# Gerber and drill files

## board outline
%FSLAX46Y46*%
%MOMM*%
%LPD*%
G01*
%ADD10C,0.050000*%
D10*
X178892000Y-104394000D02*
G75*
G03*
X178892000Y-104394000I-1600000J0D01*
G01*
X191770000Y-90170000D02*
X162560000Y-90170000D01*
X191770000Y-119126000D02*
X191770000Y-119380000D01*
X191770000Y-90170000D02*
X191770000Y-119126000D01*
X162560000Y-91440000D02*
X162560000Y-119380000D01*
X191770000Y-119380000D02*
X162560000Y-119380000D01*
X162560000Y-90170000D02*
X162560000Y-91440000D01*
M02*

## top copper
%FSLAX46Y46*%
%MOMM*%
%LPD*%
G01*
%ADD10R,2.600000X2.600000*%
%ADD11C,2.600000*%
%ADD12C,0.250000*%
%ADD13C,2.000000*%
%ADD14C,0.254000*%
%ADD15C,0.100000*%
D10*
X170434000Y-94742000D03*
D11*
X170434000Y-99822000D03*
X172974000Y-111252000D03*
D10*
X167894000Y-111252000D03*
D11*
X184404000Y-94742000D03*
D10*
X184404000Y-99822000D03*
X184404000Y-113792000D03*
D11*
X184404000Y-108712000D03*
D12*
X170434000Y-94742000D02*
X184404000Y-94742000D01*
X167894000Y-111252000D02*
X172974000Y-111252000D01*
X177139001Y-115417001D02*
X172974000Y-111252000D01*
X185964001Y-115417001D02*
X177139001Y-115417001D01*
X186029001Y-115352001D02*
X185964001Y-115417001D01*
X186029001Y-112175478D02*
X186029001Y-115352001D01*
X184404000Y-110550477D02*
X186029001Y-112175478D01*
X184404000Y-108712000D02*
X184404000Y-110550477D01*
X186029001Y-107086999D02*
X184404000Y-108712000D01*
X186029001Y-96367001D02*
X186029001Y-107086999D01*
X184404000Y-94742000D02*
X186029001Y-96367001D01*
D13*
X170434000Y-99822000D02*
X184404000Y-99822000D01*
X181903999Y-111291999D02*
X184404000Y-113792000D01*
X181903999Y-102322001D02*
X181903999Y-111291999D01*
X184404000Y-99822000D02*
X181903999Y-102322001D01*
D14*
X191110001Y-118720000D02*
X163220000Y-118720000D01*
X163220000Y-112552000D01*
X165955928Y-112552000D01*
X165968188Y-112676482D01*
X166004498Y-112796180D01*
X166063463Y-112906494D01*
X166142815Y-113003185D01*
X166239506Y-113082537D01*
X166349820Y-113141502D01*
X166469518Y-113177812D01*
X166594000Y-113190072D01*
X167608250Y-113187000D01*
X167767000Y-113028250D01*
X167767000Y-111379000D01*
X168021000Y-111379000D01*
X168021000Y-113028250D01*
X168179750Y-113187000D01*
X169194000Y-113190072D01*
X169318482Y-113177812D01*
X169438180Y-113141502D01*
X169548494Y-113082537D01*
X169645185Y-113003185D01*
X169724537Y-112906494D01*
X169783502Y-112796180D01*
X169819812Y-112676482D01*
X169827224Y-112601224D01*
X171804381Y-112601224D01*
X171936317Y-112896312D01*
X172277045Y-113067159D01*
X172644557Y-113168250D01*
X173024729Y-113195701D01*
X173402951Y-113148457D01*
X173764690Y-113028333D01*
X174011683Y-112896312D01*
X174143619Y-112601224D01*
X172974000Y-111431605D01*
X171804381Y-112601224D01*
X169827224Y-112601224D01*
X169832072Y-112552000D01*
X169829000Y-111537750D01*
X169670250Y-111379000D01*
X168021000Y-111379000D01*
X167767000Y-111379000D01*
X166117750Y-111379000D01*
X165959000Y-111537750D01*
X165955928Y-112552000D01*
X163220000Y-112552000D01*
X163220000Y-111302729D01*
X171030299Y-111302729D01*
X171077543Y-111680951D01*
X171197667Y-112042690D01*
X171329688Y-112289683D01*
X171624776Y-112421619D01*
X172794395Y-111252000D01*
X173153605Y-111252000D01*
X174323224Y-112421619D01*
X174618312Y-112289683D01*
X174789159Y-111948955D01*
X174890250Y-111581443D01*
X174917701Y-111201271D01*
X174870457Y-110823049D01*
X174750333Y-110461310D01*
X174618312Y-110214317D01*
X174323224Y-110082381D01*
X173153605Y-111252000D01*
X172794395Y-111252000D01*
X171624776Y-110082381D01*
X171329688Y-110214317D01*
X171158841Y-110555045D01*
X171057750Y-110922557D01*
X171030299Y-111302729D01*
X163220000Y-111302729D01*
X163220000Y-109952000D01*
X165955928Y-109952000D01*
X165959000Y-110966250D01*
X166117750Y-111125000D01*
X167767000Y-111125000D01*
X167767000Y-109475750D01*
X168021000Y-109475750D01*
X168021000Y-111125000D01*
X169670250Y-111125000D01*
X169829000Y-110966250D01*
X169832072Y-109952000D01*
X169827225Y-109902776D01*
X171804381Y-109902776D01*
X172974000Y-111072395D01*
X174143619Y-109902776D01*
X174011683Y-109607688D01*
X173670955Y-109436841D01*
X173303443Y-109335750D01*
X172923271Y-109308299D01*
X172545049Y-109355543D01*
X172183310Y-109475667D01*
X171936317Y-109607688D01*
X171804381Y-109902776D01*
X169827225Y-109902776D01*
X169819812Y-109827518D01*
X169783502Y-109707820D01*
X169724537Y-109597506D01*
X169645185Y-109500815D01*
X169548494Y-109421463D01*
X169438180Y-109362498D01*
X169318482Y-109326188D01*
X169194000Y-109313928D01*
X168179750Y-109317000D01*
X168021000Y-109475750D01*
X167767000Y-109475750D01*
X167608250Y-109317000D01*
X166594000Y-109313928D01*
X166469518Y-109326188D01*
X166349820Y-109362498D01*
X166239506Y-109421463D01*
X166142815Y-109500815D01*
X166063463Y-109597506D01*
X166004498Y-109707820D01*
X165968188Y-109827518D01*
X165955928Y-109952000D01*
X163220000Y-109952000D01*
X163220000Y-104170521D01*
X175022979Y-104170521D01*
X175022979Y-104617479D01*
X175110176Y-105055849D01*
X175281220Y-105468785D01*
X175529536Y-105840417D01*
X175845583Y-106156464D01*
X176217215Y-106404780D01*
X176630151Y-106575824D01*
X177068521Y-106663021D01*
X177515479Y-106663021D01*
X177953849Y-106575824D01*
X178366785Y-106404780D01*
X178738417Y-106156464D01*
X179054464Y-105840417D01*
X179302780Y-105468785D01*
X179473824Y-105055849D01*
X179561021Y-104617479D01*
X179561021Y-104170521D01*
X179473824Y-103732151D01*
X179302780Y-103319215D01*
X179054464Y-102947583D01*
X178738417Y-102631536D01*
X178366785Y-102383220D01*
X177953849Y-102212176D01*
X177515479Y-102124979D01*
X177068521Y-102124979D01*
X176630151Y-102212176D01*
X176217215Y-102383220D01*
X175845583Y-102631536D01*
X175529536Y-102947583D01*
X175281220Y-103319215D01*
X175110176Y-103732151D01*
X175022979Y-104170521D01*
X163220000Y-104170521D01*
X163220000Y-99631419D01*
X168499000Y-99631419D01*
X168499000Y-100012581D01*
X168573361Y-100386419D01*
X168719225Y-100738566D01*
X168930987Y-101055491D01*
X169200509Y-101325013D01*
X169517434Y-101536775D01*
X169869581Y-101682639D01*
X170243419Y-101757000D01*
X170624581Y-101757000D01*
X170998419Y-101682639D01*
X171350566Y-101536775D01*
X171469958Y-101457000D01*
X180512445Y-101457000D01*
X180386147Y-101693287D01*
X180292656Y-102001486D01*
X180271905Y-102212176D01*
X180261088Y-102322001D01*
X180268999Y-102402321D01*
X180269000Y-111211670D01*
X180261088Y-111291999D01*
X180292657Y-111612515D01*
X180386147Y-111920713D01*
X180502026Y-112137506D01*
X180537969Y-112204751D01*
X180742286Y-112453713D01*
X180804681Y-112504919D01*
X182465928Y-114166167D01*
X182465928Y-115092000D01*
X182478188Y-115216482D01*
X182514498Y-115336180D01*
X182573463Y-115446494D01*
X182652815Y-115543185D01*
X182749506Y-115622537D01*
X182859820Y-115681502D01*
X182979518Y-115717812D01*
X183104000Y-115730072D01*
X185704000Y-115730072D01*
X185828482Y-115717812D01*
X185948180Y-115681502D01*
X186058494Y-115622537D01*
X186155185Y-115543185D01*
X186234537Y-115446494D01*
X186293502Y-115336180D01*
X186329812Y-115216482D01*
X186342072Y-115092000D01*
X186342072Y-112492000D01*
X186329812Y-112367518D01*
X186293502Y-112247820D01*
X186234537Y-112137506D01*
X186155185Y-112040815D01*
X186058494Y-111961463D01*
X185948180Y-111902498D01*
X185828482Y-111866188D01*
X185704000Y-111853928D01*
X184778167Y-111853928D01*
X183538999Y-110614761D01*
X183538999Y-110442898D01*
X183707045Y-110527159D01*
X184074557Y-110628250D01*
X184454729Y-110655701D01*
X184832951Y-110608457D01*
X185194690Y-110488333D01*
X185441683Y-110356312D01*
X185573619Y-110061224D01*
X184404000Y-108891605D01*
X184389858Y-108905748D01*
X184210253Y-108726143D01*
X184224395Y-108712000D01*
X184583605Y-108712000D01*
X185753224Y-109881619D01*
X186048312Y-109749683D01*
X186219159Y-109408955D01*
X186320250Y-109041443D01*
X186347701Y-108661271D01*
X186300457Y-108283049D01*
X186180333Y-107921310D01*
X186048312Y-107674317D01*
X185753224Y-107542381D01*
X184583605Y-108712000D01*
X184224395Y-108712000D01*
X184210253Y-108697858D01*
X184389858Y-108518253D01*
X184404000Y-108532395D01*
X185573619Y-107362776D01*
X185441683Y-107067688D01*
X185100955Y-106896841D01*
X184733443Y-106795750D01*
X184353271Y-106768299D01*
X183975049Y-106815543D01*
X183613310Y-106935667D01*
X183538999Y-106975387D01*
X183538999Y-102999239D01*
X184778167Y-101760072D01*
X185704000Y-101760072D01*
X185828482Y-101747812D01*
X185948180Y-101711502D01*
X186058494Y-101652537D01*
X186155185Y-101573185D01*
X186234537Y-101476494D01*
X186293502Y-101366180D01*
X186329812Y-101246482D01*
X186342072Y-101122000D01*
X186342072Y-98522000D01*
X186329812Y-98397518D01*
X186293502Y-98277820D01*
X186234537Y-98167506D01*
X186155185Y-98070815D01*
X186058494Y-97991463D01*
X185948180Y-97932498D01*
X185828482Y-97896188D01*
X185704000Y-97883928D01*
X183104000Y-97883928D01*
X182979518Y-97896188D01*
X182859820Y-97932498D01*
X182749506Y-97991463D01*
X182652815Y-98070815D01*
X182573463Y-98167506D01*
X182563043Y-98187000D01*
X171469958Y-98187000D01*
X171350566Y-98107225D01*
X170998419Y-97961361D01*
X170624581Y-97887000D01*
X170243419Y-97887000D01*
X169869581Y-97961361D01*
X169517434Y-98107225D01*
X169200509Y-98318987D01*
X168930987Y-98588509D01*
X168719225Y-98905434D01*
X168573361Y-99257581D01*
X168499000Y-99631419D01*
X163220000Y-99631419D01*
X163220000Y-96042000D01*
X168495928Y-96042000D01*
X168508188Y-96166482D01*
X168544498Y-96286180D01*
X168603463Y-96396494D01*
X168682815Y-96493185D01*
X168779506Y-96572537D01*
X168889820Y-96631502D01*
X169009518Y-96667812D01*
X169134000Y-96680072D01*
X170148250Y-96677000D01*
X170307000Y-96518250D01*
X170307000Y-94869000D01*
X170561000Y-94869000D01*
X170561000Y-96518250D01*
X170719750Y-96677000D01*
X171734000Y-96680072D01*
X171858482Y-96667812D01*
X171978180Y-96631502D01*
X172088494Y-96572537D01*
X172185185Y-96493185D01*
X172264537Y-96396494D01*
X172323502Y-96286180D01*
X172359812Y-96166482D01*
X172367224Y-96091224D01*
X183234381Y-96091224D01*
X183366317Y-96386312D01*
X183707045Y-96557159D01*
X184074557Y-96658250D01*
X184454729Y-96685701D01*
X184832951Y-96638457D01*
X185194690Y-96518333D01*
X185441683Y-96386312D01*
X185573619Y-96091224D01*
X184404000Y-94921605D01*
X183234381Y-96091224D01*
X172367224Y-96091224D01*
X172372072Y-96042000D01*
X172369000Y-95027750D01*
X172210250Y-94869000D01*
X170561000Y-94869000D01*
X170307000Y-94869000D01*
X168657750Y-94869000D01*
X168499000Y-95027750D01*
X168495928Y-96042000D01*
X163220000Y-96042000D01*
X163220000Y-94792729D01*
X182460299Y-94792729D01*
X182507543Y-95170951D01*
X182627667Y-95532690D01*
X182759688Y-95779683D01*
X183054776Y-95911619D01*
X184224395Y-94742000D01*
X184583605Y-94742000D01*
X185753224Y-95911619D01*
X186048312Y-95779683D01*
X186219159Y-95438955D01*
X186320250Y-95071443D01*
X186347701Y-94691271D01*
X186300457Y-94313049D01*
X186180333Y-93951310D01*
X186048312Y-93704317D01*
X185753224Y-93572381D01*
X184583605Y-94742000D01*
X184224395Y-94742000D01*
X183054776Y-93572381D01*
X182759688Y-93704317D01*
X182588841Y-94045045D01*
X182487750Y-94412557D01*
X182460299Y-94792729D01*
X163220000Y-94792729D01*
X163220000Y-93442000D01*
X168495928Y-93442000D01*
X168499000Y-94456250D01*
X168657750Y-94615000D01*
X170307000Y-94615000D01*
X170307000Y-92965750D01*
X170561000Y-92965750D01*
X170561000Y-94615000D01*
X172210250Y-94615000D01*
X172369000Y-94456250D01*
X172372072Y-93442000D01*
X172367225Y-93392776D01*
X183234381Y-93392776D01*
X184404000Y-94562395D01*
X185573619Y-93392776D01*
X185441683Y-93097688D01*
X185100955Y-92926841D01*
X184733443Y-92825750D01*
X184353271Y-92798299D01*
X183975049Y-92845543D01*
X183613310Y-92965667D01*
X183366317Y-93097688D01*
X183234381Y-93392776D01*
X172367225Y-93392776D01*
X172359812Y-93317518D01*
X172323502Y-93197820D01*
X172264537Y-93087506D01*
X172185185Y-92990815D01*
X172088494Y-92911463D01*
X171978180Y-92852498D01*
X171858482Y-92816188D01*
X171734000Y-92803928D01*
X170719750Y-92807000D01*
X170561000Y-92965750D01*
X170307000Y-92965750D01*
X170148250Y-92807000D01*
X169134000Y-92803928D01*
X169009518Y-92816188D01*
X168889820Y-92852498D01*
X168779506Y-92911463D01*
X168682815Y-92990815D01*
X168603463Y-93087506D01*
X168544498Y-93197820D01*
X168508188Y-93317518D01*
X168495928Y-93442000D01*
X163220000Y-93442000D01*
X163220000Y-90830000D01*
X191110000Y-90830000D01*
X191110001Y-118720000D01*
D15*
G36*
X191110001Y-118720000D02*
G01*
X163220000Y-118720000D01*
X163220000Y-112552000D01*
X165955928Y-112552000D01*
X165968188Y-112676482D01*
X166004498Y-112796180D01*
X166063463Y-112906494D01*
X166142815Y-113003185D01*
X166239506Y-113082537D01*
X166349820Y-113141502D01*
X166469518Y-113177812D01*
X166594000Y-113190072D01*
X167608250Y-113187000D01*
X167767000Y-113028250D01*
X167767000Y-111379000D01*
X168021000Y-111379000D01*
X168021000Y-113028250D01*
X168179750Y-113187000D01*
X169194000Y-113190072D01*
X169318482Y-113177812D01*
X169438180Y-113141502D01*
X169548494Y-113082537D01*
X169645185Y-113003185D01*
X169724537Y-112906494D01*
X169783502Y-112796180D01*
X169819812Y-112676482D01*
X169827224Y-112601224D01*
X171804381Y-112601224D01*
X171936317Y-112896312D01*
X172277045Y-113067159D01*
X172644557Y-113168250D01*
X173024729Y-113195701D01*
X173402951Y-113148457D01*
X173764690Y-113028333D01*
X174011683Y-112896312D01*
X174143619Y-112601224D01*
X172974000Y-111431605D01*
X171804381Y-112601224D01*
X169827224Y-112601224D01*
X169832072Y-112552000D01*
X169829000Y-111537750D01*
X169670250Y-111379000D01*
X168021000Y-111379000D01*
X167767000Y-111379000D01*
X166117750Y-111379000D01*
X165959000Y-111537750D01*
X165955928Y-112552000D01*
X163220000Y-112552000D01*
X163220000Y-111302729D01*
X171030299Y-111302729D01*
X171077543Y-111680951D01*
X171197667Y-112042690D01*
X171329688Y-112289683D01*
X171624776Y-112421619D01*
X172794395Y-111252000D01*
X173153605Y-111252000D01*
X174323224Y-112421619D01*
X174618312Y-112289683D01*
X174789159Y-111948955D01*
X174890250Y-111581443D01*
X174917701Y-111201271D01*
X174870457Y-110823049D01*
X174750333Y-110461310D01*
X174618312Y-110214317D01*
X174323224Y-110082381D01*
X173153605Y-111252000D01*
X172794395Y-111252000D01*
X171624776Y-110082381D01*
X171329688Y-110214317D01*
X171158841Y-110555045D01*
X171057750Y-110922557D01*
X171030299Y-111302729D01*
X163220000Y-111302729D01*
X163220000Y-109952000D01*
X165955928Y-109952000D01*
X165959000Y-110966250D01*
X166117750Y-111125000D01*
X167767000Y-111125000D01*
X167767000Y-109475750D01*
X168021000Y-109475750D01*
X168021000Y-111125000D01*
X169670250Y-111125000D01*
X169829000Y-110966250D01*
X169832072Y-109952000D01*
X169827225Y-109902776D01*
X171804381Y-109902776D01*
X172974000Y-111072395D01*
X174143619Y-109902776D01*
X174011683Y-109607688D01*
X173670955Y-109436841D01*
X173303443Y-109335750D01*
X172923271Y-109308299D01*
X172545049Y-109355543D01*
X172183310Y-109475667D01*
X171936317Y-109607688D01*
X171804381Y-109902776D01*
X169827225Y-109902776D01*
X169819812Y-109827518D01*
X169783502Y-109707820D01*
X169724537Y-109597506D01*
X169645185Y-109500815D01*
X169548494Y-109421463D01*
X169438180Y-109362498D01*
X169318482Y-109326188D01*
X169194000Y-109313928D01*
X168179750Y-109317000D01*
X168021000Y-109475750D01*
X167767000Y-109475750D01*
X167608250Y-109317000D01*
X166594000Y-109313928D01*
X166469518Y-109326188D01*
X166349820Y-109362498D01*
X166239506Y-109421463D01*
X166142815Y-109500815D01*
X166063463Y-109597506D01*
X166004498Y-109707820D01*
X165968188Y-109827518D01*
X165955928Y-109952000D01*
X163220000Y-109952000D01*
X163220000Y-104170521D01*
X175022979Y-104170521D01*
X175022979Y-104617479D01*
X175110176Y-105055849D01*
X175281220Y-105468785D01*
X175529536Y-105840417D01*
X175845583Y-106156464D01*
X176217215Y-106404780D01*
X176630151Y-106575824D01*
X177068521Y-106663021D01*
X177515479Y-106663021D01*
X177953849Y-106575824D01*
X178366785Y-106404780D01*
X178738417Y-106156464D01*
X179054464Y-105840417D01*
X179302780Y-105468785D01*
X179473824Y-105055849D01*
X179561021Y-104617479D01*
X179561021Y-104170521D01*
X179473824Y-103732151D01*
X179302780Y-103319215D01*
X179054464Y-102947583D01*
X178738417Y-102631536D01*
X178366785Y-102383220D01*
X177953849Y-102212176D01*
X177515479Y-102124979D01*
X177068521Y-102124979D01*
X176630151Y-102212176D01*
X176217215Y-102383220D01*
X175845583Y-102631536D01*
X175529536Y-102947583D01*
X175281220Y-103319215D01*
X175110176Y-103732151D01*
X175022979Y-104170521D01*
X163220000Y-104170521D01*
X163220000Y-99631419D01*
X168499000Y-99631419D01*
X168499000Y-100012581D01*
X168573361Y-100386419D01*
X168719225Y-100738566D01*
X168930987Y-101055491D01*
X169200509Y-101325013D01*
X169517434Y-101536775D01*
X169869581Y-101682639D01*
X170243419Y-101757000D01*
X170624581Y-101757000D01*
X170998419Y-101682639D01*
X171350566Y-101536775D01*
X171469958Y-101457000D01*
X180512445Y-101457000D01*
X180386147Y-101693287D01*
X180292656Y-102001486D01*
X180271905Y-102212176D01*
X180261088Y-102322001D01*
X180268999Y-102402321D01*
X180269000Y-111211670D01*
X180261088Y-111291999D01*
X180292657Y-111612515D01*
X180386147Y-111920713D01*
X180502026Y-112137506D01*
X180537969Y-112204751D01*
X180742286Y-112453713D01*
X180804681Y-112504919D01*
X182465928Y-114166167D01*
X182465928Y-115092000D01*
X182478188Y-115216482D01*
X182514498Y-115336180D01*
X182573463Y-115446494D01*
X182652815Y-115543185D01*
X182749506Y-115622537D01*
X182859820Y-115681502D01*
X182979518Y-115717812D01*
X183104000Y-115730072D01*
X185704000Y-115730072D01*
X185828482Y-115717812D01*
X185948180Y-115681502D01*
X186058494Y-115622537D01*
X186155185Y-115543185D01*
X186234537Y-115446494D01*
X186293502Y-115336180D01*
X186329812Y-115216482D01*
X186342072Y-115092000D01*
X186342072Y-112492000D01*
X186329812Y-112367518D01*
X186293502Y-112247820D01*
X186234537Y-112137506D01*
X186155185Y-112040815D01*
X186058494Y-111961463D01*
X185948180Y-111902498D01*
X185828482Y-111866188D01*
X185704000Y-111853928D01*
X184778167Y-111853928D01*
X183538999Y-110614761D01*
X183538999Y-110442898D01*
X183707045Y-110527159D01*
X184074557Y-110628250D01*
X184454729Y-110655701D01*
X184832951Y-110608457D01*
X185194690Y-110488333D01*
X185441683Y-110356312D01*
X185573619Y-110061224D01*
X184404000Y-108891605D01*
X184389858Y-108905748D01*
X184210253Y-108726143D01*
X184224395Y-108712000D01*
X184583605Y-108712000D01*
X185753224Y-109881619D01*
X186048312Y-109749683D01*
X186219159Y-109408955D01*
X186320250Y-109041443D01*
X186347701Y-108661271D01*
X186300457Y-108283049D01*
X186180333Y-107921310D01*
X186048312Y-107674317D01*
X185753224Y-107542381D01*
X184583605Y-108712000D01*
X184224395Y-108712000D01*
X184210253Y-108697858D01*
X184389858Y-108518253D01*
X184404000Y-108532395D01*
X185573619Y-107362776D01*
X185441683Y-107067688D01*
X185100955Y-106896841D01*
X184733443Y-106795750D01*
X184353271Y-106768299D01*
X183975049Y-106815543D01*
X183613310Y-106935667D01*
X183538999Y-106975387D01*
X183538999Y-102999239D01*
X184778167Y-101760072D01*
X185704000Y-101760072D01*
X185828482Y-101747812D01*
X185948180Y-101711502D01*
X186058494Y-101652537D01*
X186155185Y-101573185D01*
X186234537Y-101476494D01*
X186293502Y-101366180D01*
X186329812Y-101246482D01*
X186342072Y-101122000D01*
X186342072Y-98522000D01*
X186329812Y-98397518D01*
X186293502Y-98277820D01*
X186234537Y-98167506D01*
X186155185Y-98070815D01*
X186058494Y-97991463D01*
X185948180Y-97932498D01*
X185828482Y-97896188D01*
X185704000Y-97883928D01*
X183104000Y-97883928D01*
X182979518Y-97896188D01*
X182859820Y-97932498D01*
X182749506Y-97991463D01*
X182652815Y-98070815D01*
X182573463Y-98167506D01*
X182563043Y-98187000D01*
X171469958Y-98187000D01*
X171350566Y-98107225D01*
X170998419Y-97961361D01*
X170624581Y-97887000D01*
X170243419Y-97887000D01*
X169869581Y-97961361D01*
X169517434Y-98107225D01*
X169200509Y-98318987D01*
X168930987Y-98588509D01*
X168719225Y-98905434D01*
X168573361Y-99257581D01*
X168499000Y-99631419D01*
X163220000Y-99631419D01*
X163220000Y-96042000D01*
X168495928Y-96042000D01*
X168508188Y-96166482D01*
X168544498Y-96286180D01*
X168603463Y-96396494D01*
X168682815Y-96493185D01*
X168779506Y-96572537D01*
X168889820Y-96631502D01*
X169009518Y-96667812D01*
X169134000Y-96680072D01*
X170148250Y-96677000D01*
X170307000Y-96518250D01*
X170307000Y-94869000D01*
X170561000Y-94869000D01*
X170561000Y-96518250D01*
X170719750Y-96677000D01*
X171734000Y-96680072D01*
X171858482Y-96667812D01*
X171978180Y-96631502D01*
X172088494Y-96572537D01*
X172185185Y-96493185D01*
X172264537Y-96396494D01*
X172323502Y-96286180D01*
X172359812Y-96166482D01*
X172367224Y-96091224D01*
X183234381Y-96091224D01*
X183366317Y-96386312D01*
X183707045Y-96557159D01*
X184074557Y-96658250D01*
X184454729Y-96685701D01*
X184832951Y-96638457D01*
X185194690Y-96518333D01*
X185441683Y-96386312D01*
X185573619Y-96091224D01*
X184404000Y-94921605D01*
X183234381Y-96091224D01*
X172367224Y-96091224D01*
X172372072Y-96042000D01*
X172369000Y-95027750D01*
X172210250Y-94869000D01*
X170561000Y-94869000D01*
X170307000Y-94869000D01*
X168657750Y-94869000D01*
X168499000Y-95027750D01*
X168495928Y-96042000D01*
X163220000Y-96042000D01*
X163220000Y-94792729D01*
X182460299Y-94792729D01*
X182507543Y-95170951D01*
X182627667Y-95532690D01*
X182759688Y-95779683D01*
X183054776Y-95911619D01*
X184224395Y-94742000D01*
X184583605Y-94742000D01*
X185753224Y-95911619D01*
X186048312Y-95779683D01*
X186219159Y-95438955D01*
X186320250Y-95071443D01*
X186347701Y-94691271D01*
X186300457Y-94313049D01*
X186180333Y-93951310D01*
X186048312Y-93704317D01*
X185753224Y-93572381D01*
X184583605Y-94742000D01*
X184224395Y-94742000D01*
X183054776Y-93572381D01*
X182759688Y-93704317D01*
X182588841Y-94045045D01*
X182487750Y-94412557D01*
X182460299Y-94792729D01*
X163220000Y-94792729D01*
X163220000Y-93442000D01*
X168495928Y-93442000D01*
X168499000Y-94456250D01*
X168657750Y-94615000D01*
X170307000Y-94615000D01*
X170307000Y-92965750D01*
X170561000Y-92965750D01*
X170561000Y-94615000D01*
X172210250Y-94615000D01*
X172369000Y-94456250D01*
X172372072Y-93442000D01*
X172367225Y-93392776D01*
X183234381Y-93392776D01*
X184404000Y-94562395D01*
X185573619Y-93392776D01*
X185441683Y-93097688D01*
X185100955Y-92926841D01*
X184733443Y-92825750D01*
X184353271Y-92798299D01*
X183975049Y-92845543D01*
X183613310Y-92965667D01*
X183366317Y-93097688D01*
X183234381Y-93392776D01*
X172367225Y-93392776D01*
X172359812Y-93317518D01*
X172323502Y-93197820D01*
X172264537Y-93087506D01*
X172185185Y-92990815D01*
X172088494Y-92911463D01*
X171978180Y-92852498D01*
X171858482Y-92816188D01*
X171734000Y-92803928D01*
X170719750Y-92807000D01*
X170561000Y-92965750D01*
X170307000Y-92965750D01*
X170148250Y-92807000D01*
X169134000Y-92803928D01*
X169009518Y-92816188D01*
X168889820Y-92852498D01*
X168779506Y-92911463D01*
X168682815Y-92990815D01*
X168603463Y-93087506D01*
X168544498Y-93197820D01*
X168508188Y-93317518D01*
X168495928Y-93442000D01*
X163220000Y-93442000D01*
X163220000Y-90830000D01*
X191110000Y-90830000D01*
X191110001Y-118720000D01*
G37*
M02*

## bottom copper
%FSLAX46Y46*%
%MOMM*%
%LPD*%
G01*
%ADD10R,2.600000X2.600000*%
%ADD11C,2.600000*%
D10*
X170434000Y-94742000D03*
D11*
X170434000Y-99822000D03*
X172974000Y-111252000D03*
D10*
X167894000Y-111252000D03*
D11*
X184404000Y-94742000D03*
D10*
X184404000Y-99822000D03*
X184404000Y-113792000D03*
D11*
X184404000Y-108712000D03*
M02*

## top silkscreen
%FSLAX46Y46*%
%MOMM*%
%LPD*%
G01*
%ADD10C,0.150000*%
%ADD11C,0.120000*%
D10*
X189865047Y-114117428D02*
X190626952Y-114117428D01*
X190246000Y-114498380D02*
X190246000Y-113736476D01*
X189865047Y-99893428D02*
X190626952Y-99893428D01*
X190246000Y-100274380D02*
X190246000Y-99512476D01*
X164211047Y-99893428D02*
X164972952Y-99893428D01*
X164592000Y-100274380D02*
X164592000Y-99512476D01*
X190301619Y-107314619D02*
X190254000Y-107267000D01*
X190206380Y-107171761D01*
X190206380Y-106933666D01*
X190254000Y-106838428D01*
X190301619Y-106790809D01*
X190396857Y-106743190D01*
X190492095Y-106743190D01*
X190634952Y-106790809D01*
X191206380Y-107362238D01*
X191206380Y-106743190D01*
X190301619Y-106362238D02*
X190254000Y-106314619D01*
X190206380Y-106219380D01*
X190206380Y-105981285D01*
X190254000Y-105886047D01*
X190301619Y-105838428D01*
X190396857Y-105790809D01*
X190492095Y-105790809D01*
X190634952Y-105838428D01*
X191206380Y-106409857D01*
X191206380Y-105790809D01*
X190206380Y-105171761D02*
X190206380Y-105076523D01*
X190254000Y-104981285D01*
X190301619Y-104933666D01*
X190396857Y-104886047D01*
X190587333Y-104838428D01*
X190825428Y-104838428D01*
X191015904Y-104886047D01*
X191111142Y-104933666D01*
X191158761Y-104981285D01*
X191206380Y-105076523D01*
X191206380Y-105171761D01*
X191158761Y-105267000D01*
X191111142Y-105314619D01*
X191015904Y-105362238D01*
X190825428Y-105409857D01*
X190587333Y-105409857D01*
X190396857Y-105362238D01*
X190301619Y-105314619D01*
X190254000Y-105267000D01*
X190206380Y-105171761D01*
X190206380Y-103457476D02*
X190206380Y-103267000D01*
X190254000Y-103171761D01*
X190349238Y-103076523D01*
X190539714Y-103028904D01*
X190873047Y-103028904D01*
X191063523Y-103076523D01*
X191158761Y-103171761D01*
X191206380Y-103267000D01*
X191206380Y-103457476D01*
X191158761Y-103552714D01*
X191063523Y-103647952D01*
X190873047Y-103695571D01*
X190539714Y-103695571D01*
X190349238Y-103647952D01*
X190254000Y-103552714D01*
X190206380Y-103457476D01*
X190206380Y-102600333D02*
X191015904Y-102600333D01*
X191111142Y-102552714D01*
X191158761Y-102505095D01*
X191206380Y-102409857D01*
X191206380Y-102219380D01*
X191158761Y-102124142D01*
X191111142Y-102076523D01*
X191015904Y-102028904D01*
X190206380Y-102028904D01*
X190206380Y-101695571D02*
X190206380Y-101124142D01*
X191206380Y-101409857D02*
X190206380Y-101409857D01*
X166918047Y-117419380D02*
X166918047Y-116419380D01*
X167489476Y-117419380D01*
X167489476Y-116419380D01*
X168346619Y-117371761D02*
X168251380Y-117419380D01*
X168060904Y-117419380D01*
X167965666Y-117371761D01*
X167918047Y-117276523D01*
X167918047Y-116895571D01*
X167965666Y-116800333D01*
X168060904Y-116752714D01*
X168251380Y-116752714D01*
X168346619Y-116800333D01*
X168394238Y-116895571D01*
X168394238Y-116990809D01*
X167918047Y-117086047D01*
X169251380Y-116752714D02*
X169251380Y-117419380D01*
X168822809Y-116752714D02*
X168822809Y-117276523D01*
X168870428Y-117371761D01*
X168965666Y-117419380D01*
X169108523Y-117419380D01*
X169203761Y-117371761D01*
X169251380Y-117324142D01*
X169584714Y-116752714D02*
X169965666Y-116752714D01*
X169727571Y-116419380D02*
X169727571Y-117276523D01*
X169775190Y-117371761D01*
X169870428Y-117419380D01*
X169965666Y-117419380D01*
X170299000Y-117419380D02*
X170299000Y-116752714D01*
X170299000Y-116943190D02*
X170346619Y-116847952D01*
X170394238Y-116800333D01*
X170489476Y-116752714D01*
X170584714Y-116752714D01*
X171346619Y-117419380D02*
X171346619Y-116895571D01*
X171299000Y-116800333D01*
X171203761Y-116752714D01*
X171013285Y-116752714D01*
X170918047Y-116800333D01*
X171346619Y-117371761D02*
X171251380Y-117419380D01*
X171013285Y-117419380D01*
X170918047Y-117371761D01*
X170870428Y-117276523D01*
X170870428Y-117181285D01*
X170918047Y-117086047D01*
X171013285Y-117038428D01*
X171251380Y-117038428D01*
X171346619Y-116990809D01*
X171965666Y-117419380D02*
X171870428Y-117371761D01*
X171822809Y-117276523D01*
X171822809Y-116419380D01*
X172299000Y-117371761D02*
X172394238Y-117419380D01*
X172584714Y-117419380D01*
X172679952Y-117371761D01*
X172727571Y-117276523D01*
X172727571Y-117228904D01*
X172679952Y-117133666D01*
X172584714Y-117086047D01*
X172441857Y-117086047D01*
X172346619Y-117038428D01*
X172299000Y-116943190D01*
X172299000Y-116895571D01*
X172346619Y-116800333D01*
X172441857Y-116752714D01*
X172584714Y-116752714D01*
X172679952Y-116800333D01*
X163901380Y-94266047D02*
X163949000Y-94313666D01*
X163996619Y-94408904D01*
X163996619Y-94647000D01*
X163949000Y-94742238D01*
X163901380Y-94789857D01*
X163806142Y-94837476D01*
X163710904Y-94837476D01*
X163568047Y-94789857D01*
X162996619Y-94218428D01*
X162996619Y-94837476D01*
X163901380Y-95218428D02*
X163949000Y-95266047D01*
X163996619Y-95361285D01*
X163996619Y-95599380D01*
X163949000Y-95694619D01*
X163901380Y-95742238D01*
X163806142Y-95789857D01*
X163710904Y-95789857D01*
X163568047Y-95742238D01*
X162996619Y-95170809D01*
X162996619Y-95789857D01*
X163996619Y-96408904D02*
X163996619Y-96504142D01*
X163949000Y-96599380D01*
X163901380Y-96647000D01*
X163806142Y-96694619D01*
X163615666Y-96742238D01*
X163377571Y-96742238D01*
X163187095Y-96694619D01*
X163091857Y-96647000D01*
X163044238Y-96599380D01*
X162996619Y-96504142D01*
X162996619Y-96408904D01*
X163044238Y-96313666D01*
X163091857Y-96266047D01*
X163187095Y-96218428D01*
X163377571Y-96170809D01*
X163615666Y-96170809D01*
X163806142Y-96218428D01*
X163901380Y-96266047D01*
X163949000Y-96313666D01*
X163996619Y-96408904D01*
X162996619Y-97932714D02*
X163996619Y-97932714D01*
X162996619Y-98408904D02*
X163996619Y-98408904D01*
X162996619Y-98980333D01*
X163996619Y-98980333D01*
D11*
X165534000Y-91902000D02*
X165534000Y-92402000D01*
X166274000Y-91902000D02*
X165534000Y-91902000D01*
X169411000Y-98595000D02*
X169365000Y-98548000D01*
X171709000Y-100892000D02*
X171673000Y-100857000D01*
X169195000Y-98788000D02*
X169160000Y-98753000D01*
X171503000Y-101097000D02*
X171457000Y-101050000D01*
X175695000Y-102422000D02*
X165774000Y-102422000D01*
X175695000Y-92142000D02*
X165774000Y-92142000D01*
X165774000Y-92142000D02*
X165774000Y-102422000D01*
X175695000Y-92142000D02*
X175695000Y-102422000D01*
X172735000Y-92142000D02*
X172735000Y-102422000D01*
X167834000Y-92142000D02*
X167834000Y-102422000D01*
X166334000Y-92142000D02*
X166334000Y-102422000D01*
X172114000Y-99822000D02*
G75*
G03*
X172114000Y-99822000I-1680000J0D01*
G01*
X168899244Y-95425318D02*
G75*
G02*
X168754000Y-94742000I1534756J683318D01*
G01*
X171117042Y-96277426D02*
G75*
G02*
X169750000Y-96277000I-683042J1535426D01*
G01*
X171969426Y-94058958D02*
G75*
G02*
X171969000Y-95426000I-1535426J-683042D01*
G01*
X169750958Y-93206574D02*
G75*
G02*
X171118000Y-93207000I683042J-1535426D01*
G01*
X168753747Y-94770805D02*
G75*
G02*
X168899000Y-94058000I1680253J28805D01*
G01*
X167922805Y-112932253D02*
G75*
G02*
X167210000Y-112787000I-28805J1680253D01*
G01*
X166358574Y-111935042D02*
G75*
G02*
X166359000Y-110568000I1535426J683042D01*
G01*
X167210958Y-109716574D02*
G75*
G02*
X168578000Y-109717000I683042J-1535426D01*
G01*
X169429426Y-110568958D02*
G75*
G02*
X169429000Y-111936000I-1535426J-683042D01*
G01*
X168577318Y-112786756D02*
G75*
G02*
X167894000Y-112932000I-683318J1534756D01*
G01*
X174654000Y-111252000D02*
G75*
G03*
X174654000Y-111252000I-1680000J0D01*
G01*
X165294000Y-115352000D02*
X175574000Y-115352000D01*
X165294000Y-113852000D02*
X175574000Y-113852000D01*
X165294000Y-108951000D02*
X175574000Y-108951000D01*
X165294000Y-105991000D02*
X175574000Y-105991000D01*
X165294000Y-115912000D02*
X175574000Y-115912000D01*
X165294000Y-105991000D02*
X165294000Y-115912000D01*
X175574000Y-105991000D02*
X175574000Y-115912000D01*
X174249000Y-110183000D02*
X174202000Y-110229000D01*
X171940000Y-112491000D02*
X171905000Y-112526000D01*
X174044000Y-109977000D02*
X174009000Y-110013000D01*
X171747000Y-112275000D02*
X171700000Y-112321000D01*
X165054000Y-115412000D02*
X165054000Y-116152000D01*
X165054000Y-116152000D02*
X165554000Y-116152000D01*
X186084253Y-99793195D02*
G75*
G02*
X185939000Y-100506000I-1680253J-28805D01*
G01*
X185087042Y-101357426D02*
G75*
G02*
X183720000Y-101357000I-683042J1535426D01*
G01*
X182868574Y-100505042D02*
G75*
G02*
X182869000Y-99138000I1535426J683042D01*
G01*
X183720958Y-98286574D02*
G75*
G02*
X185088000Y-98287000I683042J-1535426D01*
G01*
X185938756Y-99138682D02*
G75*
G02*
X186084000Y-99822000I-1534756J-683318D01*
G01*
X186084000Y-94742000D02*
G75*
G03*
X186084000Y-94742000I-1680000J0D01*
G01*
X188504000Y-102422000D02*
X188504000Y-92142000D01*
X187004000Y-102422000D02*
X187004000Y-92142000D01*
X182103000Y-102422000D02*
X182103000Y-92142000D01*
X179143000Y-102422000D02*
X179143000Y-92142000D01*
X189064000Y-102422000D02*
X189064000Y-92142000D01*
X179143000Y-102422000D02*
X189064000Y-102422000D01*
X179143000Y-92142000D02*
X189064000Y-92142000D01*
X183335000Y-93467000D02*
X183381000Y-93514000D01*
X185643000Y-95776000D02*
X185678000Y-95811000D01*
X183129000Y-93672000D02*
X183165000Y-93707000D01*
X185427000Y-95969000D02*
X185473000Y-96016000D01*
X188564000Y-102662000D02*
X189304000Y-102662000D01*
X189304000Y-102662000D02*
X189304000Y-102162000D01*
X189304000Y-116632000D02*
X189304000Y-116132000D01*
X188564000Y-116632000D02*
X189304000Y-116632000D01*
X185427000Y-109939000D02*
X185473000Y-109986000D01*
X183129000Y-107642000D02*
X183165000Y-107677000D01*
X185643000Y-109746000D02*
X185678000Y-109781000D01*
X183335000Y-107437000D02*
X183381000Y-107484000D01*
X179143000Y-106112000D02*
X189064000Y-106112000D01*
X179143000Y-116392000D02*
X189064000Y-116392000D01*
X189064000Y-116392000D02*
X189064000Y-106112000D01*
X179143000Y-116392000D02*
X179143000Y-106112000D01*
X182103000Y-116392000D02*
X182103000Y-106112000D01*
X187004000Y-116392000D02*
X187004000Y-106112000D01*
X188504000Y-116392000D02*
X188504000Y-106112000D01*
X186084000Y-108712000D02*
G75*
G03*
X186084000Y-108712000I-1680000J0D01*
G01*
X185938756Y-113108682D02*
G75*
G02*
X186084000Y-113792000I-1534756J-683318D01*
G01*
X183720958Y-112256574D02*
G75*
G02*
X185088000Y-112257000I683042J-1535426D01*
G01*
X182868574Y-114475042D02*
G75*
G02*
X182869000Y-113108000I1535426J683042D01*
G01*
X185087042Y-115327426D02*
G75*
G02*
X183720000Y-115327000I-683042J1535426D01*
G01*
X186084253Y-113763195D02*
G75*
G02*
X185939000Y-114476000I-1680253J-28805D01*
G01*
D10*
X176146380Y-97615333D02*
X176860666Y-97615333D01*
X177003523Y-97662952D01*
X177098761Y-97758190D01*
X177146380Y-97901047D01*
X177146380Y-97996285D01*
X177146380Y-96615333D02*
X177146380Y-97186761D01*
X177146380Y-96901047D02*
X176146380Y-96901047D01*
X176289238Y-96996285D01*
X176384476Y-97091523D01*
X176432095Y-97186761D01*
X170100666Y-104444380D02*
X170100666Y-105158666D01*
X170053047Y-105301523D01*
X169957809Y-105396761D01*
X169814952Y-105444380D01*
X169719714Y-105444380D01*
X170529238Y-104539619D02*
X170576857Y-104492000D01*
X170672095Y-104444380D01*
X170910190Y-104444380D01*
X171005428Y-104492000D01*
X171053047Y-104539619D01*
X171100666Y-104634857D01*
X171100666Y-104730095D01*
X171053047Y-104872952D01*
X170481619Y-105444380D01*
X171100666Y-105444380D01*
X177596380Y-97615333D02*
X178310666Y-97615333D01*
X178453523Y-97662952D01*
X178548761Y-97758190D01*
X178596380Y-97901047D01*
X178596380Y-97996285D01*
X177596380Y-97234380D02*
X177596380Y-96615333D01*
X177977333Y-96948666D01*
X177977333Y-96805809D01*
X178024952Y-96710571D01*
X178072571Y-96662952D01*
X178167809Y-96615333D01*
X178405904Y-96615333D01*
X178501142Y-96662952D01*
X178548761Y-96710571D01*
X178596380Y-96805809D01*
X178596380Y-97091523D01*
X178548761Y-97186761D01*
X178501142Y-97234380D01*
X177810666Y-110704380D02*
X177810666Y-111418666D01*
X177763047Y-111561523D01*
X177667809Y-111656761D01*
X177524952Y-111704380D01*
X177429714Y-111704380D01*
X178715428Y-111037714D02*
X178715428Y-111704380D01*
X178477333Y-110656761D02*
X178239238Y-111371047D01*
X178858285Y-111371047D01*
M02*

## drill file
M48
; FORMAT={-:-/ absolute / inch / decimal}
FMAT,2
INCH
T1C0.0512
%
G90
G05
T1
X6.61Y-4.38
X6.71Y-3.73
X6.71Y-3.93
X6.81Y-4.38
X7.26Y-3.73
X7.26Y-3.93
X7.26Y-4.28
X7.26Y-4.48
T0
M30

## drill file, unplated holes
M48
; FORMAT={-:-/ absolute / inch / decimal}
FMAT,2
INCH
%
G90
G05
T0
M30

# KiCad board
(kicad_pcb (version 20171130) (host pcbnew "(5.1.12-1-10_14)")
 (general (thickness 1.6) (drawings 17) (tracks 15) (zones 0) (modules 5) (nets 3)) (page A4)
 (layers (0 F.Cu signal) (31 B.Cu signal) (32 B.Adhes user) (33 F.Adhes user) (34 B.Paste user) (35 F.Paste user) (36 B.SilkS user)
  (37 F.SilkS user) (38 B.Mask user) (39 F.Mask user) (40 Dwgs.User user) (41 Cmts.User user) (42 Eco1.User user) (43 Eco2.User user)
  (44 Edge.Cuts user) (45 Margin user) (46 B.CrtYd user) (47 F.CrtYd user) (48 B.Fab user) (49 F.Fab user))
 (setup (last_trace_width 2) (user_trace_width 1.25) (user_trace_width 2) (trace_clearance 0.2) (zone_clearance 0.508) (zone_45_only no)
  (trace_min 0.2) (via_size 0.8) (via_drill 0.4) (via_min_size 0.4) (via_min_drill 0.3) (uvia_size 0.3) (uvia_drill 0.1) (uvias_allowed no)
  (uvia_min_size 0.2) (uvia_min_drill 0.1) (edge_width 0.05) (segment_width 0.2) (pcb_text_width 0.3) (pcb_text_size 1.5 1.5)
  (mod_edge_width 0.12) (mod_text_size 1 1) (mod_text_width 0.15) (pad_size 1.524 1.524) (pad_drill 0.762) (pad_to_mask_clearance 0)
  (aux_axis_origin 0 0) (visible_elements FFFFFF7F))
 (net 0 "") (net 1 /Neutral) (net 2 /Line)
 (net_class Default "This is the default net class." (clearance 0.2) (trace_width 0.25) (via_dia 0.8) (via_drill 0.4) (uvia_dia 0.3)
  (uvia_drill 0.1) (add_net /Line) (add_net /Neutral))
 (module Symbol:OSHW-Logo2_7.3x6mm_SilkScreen (layer B.Cu) (at 178.054 111.252 180)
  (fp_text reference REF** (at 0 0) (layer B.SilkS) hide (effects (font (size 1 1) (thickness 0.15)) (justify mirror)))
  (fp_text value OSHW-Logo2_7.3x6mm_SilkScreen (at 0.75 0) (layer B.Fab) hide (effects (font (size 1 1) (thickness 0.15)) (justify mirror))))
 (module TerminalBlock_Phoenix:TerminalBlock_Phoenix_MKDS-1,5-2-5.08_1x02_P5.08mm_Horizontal (layer F.Cu) (at 170.434 94.742 270)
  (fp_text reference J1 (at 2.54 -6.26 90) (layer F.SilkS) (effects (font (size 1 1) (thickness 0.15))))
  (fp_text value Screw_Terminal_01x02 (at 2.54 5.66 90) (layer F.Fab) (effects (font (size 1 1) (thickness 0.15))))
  (fp_line (start -2.84 4.9) (end -2.34 4.9) (layer F.SilkS) (width 0.12))
  (fp_line (start -2.84 4.16) (end -2.84 4.9) (layer F.SilkS) (width 0.12))
  (fp_line (start 3.853 1.023) (end 3.806 1.069) (layer F.SilkS) (width 0.12))
  (fp_line (start 6.15 -1.275) (end 6.115 -1.239) (layer F.SilkS) (width 0.12))
  (fp_line (start 4.046 1.239) (end 4.011 1.274) (layer F.SilkS) (width 0.12))
  (fp_line (start 6.355 -1.069) (end 6.308 -1.023) (layer F.SilkS) (width 0.12))
  (fp_line (start 7.68 -5.261) (end 7.68 4.66) (layer F.SilkS) (width 0.12))
  (fp_line (start -2.6 -5.261) (end -2.6 4.66) (layer F.SilkS) (width 0.12))
  (fp_line (start -2.6 4.66) (end 7.68 4.66) (layer F.SilkS) (width 0.12))
  (fp_line (start -2.6 -5.261) (end 7.68 -5.261) (layer F.SilkS) (width 0.12))
  (fp_line (start -2.6 -2.301) (end 7.68 -2.301) (layer F.SilkS) (width 0.12))
  (fp_line (start -2.6 2.6) (end 7.68 2.6) (layer F.SilkS) (width 0.12))
  (fp_line (start -2.6 4.1) (end 7.68 4.1) (layer F.SilkS) (width 0.12))
  (fp_circle (center 5.08 0) (end 6.76 0) (layer F.SilkS) (width 0.12))
  (fp_arc (start 0 0) (end 0 1.68) (angle -24) (layer F.SilkS) (width 0.12))
  (fp_arc (start 0 0) (end 1.535 0.684) (angle -48) (layer F.SilkS) (width 0.12))
  (fp_arc (start 0 0) (end 0.684 -1.535) (angle -48) (layer F.SilkS) (width 0.12))
  (fp_arc (start 0 0) (end -1.535 -0.684) (angle -48) (layer F.SilkS) (width 0.12))
  (fp_arc (start 0 0) (end -0.684 1.535) (angle -25) (layer F.SilkS) (width 0.12))
  (pad 1 thru_hole rect (at 0 0 270) (size 2.6 2.6) (drill 1.3) (layers *.Cu *.Mask) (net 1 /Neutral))
  (pad 2 thru_hole circle (at 5.08 0 270) (size 2.6 2.6) (drill 1.3) (layers *.Cu *.Mask) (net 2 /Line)))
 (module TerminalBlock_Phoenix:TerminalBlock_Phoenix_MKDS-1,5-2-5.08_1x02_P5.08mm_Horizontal (layer F.Cu) (at 167.894 111.252)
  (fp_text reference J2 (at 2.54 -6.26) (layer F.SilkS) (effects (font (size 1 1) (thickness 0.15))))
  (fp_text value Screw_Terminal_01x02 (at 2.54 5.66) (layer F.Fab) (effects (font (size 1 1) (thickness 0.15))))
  (fp_arc (start 0 0) (end -0.684 1.535) (angle -25) (layer F.SilkS) (width 0.12))
  (fp_arc (start 0 0) (end -1.535 -0.684) (angle -48) (layer F.SilkS) (width 0.12))
  (fp_arc (start 0 0) (end 0.684 -1.535) (angle -48) (layer F.SilkS) (width 0.12))
  (fp_arc (start 0 0) (end 1.535 0.684) (angle -48) (layer F.SilkS) (width 0.12))
  (fp_arc (start 0 0) (end 0 1.68) (angle -24) (layer F.SilkS) (width 0.12))
  (fp_circle (center 5.08 0) (end 6.76 0) (layer F.SilkS) (width 0.12))
  (fp_line (start -2.6 4.1) (end 7.68 4.1) (layer F.SilkS) (width 0.12))
  (fp_line (start -2.6 2.6) (end 7.68 2.6) (layer F.SilkS) (width 0.12))
  (fp_line (start -2.6 -2.301) (end 7.68 -2.301) (layer F.SilkS) (width 0.12))
  (fp_line (start -2.6 -5.261) (end 7.68 -5.261) (layer F.SilkS) (width 0.12))
  (fp_line (start -2.6 4.66) (end 7.68 4.66) (layer F.SilkS) (width 0.12))
  (fp_line (start -2.6 -5.261) (end -2.6 4.66) (layer F.SilkS) (width 0.12))
  (fp_line (start 7.68 -5.261) (end 7.68 4.66) (layer F.SilkS) (width 0.12))
  (fp_line (start 6.355 -1.069) (end 6.308 -1.023) (layer F.SilkS) (width 0.12))
  (fp_line (start 4.046 1.239) (end 4.011 1.274) (layer F.SilkS) (width 0.12))
  (fp_line (start 6.15 -1.275) (end 6.115 -1.239) (layer F.SilkS) (width 0.12))
  (fp_line (start 3.853 1.023) (end 3.806 1.069) (layer F.SilkS) (width 0.12))
  (fp_line (start -2.84 4.16) (end -2.84 4.9) (layer F.SilkS) (width 0.12))
  (fp_line (start -2.84 4.9) (end -2.34 4.9) (layer F.SilkS) (width 0.12))
  (pad 2 thru_hole circle (at 5.08 0) (size 2.6 2.6) (drill 1.3) (layers *.Cu *.Mask) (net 1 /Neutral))
  (pad 1 thru_hole rect (at 0 0) (size 2.6 2.6) (drill 1.3) (layers *.Cu *.Mask) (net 1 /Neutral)))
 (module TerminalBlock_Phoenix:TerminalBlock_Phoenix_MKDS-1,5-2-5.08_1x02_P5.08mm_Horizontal (layer F.Cu) (at 184.404 99.822 90)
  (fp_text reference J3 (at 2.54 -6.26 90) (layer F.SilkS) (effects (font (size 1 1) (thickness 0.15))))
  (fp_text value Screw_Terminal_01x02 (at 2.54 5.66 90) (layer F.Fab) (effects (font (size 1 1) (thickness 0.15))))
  (fp_arc (start 0 0) (end -0.684 1.535) (angle -25) (layer F.SilkS) (width 0.12))
  (fp_arc (start 0 0) (end -1.535 -0.684) (angle -48) (layer F.SilkS) (width 0.12))
  (fp_arc (start 0 0) (end 0.684 -1.535) (angle -48) (layer F.SilkS) (width 0.12))
  (fp_arc (start 0 0) (end 1.535 0.684) (angle -48) (layer F.SilkS) (width 0.12))
  (fp_arc (start 0 0) (end 0 1.68) (angle -24) (layer F.SilkS) (width 0.12))
  (fp_circle (center 5.08 0) (end 6.76 0) (layer F.SilkS) (width 0.12))
  (fp_line (start -2.6 4.1) (end 7.68 4.1) (layer F.SilkS) (width 0.12))
  (fp_line (start -2.6 2.6) (end 7.68 2.6) (layer F.SilkS) (width 0.12))
  (fp_line (start -2.6 -2.301) (end 7.68 -2.301) (layer F.SilkS) (width 0.12))
  (fp_line (start -2.6 -5.261) (end 7.68 -5.261) (layer F.SilkS) (width 0.12))
  (fp_line (start -2.6 4.66) (end 7.68 4.66) (layer F.SilkS) (width 0.12))
  (fp_line (start -2.6 -5.261) (end -2.6 4.66) (layer F.SilkS) (width 0.12))
  (fp_line (start 7.68 -5.261) (end 7.68 4.66) (layer F.SilkS) (width 0.12))
  (fp_line (start 6.355 -1.069) (end 6.308 -1.023) (layer F.SilkS) (width 0.12))
  (fp_line (start 4.046 1.239) (end 4.011 1.274) (layer F.SilkS) (width 0.12))
  (fp_line (start 6.15 -1.275) (end 6.115 -1.239) (layer F.SilkS) (width 0.12))
  (fp_line (start 3.853 1.023) (end 3.806 1.069) (layer F.SilkS) (width 0.12))
  (fp_line (start -2.84 4.16) (end -2.84 4.9) (layer F.SilkS) (width 0.12))
  (fp_line (start -2.84 4.9) (end -2.34 4.9) (layer F.SilkS) (width 0.12))
  (pad 2 thru_hole circle (at 5.08 0 90) (size 2.6 2.6) (drill 1.3) (layers *.Cu *.Mask) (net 1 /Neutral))
  (pad 1 thru_hole rect (at 0 0 90) (size 2.6 2.6) (drill 1.3) (layers *.Cu *.Mask) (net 2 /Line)))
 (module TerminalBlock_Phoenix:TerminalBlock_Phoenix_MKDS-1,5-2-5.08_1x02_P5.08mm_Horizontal (layer F.Cu) (at 184.404 113.792 90)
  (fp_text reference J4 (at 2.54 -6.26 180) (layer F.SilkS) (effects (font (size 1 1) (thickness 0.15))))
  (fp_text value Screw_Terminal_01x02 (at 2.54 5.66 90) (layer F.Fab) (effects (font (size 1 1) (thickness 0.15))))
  (fp_line (start -2.84 4.9) (end -2.34 4.9) (layer F.SilkS) (width 0.12))
  (fp_line (start -2.84 4.16) (end -2.84 4.9) (layer F.SilkS) (width 0.12))
  (fp_line (start 3.853 1.023) (end 3.806 1.069) (layer F.SilkS) (width 0.12))
  (fp_line (start 6.15 -1.275) (end 6.115 -1.239) (layer F.SilkS) (width 0.12))
  (fp_line (start 4.046 1.239) (end 4.011 1.274) (layer F.SilkS) (width 0.12))
  (fp_line (start 6.355 -1.069) (end 6.308 -1.023) (layer F.SilkS) (width 0.12))
  (fp_line (start 7.68 -5.261) (end 7.68 4.66) (layer F.SilkS) (width 0.12))
  (fp_line (start -2.6 -5.261) (end -2.6 4.66) (layer F.SilkS) (width 0.12))
  (fp_line (start -2.6 4.66) (end 7.68 4.66) (layer F.SilkS) (width 0.12))
  (fp_line (start -2.6 -5.261) (end 7.68 -5.261) (layer F.SilkS) (width 0.12))
  (fp_line (start -2.6 -2.301) (end 7.68 -2.301) (layer F.SilkS) (width 0.12))
  (fp_line (start -2.6 2.6) (end 7.68 2.6) (layer F.SilkS) (width 0.12))
  (fp_line (start -2.6 4.1) (end 7.68 4.1) (layer F.SilkS) (width 0.12))
  (fp_circle (center 5.08 0) (end 6.76 0) (layer F.SilkS) (width 0.12))
  (fp_arc (start 0 0) (end 0 1.68) (angle -24) (layer F.SilkS) (width 0.12))
  (fp_arc (start 0 0) (end 1.535 0.684) (angle -48) (layer F.SilkS) (width 0.12))
  (fp_arc (start 0 0) (end 0.684 -1.535) (angle -48) (layer F.SilkS) (width 0.12))
  (fp_arc (start 0 0) (end -1.535 -0.684) (angle -48) (layer F.SilkS) (width 0.12))
  (fp_arc (start 0 0) (end -0.684 1.535) (angle -25) (layer F.SilkS) (width 0.12))
  (pad 1 thru_hole rect (at 0 0 90) (size 2.6 2.6) (drill 1.3) (layers *.Cu *.Mask) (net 2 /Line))
  (pad 2 thru_hole circle (at 5.08 0 90) (size 2.6 2.6) (drill 1.3) (layers *.Cu *.Mask) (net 1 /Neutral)))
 (gr_circle (center 177.292 104.394) (end 178.892 104.394) (layer Edge.Cuts) (width 0.05))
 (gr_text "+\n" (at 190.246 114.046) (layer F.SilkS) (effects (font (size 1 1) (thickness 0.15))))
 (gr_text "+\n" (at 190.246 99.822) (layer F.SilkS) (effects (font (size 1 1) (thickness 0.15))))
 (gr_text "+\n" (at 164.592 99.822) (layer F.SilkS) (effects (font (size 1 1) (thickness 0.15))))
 (gr_line (start 191.77 90.17) (end 162.56 90.17) (layer Edge.Cuts) (width 0.05))
 (gr_line (start 191.77 119.126) (end 191.77 119.38) (layer Edge.Cuts) (width 0.05))
 (gr_line (start 191.77 90.17) (end 191.77 119.126) (layer Edge.Cuts) (width 0.05))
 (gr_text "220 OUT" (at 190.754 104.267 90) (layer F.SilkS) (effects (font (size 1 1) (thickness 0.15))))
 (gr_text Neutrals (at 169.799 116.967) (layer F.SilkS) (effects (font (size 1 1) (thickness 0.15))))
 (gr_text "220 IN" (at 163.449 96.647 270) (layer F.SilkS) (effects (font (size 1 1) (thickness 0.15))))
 (gr_line (start 162.56 91.44) (end 162.56 119.38) (layer Edge.Cuts) (width 0.05))
 (gr_line (start 191.77 119.38) (end 162.56 119.38) (layer Edge.Cuts) (width 0.05))
 (gr_line (start 162.56 90.17) (end 162.56 91.44) (layer Edge.Cuts) (width 0.05))
 (segment (start 170.434 94.742) (end 184.404 94.742) (width 0.25) (layer F.Cu) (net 1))
 (segment (start 167.894 111.252) (end 172.974 111.252) (width 0.25) (layer F.Cu) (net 1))
 (segment (start 177.139001 115.417001) (end 172.974 111.252) (width 0.25) (layer F.Cu) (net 1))
 (segment (start 185.964001 115.417001) (end 177.139001 115.417001) (width 0.25) (layer F.Cu) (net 1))
 (segment (start 186.029001 115.352001) (end 185.964001 115.417001) (width 0.25) (layer F.Cu) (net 1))
 (segment (start 186.029001 112.175478) (end 186.029001 115.352001) (width 0.25) (layer F.Cu) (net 1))
 (segment (start 184.404 110.550477) (end 186.029001 112.175478) (width 0.25) (layer F.Cu) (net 1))
 (segment (start 184.404 108.712) (end 184.404 110.550477) (width 0.25) (layer F.Cu) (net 1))
 (segment (start 186.029001 107.086999) (end 184.404 108.712) (width 0.25) (layer F.Cu) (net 1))
 (segment (start 186.029001 96.367001) (end 186.029001 107.086999) (width 0.25) (layer F.Cu) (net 1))
 (segment (start 184.404 94.742) (end 186.029001 96.367001) (width 0.25) (layer F.Cu) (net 1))
 (segment (start 170.434 99.822) (end 184.404 99.822) (width 2) (layer F.Cu) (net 2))
 (segment (start 181.903999 111.291999) (end 184.404 113.792) (width 2) (layer F.Cu) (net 2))
 (segment (start 181.903999 102.322001) (end 181.903999 111.291999) (width 2) (layer F.Cu) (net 2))
 (segment (start 184.404 99.822) (end 181.903999 102.322001) (width 2) (layer F.Cu) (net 2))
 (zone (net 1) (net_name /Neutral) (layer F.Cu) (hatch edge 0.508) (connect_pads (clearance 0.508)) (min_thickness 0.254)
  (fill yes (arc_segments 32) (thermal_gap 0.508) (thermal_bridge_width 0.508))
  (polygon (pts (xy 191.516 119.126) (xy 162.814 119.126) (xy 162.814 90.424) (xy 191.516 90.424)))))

